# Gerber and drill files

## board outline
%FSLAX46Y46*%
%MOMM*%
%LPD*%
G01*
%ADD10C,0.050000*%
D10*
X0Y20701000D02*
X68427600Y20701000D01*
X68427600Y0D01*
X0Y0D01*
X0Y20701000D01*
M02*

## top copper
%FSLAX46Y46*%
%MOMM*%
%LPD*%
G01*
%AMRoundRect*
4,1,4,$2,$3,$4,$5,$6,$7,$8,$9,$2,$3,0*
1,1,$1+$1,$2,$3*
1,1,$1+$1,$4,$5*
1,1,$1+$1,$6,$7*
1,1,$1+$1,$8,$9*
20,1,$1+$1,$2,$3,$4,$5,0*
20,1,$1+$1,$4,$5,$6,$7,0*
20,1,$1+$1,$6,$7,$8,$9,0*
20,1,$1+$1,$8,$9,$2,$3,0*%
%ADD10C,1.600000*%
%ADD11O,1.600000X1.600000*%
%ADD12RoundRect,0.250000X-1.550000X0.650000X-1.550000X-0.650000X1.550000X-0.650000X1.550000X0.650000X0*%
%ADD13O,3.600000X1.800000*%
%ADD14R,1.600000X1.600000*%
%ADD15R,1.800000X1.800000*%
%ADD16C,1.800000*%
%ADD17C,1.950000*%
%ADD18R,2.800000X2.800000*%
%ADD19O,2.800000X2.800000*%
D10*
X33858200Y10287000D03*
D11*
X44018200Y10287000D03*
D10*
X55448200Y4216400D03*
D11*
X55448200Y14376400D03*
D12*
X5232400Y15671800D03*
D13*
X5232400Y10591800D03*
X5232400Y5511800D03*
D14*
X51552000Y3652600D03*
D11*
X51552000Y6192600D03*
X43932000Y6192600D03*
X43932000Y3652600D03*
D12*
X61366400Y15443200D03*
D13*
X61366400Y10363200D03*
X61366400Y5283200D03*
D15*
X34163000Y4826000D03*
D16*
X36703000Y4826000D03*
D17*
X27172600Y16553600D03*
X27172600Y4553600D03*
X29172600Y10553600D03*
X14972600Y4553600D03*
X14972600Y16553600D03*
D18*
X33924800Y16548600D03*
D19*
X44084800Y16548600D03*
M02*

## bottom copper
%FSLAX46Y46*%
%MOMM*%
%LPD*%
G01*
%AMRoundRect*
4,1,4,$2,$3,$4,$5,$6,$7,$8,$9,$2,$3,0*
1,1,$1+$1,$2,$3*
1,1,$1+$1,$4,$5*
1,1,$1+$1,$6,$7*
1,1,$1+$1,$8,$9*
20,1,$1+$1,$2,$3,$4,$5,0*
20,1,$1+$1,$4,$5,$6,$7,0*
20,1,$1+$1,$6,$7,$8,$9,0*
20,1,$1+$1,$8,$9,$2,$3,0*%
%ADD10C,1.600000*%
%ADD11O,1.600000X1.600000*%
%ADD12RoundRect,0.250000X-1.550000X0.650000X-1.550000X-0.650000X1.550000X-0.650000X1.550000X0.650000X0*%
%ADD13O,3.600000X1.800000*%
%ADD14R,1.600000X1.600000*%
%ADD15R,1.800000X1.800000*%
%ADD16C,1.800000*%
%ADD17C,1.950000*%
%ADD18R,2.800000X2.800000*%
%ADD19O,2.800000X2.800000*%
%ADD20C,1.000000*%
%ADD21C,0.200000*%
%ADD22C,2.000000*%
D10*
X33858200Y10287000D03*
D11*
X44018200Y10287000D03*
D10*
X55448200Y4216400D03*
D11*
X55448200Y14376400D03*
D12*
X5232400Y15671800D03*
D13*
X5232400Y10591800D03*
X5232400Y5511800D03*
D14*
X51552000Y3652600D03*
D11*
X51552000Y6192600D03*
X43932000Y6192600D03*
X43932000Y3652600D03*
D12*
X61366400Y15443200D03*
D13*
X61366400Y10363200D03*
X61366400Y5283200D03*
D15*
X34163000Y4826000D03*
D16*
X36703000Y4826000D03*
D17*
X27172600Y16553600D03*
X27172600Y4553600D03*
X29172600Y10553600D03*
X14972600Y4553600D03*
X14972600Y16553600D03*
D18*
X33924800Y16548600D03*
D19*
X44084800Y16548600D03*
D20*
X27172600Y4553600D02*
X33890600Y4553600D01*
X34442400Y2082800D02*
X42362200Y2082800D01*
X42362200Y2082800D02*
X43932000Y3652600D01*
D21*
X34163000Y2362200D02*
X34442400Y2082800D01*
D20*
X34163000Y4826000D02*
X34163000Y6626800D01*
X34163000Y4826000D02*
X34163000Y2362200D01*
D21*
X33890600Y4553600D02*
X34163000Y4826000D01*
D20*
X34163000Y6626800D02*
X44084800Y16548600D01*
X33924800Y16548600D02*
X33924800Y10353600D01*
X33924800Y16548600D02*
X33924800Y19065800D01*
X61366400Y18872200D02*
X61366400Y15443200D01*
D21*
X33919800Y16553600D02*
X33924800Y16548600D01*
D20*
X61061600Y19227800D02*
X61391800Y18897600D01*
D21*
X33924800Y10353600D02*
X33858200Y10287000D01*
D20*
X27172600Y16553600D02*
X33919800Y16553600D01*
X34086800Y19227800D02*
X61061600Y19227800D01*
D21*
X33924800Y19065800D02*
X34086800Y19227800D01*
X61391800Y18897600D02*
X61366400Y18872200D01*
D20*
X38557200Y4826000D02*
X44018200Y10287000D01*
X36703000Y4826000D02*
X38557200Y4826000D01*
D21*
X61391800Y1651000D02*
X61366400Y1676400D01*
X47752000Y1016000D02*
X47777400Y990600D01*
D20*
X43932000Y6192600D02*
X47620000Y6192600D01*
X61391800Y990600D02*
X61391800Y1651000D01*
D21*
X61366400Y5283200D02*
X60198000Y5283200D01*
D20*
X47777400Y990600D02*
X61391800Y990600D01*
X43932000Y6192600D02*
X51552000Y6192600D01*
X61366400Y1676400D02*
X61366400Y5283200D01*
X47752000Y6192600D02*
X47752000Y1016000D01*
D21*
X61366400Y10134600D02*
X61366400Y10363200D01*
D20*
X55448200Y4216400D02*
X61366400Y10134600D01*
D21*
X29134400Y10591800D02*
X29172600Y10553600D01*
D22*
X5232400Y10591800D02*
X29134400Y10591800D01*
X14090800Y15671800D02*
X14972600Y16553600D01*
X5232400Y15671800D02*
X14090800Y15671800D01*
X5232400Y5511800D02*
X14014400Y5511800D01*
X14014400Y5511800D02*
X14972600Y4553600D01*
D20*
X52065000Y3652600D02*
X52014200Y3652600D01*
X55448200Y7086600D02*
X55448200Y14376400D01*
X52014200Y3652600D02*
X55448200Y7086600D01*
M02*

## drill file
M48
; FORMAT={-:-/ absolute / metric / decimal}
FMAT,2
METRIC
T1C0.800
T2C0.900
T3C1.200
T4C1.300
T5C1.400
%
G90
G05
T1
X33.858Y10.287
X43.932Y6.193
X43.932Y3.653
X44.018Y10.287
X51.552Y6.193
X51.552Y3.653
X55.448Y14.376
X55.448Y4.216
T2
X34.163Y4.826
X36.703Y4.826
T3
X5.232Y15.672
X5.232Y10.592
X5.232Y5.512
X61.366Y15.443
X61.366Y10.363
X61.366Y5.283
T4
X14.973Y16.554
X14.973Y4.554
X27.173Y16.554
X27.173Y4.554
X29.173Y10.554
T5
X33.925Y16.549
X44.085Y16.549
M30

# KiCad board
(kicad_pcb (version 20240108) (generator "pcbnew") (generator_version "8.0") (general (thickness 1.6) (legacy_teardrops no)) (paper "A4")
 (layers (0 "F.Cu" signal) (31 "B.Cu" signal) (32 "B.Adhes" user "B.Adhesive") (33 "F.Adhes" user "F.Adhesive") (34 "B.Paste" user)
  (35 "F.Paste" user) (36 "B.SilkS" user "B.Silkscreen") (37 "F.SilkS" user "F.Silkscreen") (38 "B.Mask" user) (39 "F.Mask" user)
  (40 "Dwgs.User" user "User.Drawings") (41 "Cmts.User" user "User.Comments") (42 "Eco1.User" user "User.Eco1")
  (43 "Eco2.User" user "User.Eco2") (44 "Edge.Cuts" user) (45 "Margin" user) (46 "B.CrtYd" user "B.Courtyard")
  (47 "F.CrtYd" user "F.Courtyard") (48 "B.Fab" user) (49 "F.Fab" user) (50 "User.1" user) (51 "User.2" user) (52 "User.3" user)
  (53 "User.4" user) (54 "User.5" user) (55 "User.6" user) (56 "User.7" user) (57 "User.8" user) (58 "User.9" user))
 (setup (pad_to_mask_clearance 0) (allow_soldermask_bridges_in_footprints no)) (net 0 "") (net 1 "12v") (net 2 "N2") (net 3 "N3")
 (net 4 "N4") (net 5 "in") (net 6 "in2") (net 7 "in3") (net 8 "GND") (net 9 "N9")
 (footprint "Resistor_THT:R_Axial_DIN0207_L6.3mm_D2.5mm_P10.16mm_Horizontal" (layer "F.Cu") (at 33.8582 -10.287)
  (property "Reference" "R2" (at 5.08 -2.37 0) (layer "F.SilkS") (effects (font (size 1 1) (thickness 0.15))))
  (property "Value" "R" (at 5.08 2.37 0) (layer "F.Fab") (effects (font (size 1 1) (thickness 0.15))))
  (pad "1" thru_hole circle (at 0 0) (size 1.6 1.6) (drill 0.8) (layers "*.Cu" "*.Mask") (remove_unused_layers no) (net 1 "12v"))
  (pad "2" thru_hole oval (at 10.16 0) (size 1.6 1.6) (drill 0.8) (layers "*.Cu" "*.Mask") (remove_unused_layers no) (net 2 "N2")))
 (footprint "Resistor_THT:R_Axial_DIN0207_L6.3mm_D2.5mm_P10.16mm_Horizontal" (layer "F.Cu") (at 55.4482 -4.2164 90)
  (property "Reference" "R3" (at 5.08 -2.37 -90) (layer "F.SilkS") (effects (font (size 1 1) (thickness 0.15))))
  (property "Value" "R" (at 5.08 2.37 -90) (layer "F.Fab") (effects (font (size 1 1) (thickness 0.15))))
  (pad "1" thru_hole circle (at 0 0 90) (size 1.6 1.6) (drill 0.8) (layers "*.Cu" "*.Mask") (remove_unused_layers no) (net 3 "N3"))
  (pad "2" thru_hole oval (at 10.16 0 90) (size 1.6 1.6) (drill 0.8) (layers "*.Cu" "*.Mask") (remove_unused_layers no) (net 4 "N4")))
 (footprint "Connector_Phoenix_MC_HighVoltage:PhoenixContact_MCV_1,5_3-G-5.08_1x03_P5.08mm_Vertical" (layer "F.Cu") (at 5.2324 -15.6718 -90)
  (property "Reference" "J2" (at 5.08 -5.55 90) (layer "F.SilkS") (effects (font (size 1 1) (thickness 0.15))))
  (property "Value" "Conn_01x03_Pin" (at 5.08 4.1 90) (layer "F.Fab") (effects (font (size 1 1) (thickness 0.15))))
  (pad "1" thru_hole roundrect (at 0 0 270) (size 1.8 3.6) (drill 1.2) (layers "*.Cu" "*.Mask") (remove_unused_layers no)
   (roundrect_rratio 0.138889) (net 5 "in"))
  (pad "2" thru_hole oval (at 5.08 0 270) (size 1.8 3.6) (drill 1.2) (layers "*.Cu" "*.Mask") (remove_unused_layers no) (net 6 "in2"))
  (pad "3" thru_hole oval (at 10.16 0 270) (size 1.8 3.6) (drill 1.2) (layers "*.Cu" "*.Mask") (remove_unused_layers no) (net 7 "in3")))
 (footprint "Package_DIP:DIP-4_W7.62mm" (layer "F.Cu") (at 51.552 -3.6526 180)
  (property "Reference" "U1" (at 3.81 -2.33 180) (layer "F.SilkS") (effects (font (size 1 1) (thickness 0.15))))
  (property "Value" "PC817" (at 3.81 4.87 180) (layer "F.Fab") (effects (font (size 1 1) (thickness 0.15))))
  (pad "1" thru_hole rect (at 0 0 180) (size 1.6 1.6) (drill 0.8) (layers "*.Cu" "*.Mask") (remove_unused_layers no) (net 4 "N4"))
  (pad "2" thru_hole oval (at 0 2.54 180) (size 1.6 1.6) (drill 0.8) (layers "*.Cu" "*.Mask") (remove_unused_layers no) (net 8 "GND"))
  (pad "3" thru_hole oval (at 7.62 2.54 180) (size 1.6 1.6) (drill 0.8) (layers "*.Cu" "*.Mask") (remove_unused_layers no) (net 8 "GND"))
  (pad "4" thru_hole oval (at 7.62 0 180) (size 1.6 1.6) (drill 0.8) (layers "*.Cu" "*.Mask") (remove_unused_layers no) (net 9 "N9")))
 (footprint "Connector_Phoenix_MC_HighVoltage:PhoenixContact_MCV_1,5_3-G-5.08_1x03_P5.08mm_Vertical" (layer "F.Cu")
  (at 61.3664 -15.4432 -90)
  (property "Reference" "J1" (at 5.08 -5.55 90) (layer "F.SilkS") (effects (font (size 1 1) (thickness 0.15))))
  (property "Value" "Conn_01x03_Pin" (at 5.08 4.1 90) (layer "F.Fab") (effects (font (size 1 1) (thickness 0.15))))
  (pad "1" thru_hole roundrect (at 0 0 270) (size 1.8 3.6) (drill 1.2) (layers "*.Cu" "*.Mask") (remove_unused_layers no)
   (roundrect_rratio 0.138889) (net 1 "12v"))
  (pad "2" thru_hole oval (at 5.08 0 270) (size 1.8 3.6) (drill 1.2) (layers "*.Cu" "*.Mask") (remove_unused_layers no) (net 3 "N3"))
  (pad "3" thru_hole oval (at 10.16 0 270) (size 1.8 3.6) (drill 1.2) (layers "*.Cu" "*.Mask") (remove_unused_layers no) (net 8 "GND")))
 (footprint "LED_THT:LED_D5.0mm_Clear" (layer "F.Cu") (at 34.163 -4.826)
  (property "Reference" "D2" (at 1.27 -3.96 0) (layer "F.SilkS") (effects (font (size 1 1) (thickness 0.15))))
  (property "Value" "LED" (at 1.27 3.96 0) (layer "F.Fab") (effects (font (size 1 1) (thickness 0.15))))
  (pad "1" thru_hole rect (at 0 0) (size 1.8 1.8) (drill 0.9) (layers "*.Cu" "*.Mask") (remove_unused_layers no) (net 9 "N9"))
  (pad "2" thru_hole circle (at 2.54 0) (size 1.8 1.8) (drill 0.9) (layers "*.Cu" "*.Mask") (remove_unused_layers no) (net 2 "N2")))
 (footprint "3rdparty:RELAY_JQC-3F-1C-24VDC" (layer "F.Cu") (at 21.0726 -10.5536)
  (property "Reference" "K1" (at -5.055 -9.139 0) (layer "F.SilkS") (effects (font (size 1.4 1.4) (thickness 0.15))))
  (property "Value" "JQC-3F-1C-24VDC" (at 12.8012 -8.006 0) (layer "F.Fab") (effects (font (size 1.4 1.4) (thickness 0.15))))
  (pad "COIL1" thru_hole circle (at 6.1 -6) (size 1.95 1.95) (drill 1.3) (layers "*.Cu" "*.Mask") (remove_unused_layers no) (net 1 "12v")
   (solder_mask_margin 0.102))
  (pad "COIL2" thru_hole circle (at 6.1 6) (size 1.95 1.95) (drill 1.3) (layers "*.Cu" "*.Mask") (remove_unused_layers no) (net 9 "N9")
   (solder_mask_margin 0.102))
  (pad "COM" thru_hole circle (at 8.1 0) (size 1.95 1.95) (drill 1.3) (layers "*.Cu" "*.Mask") (remove_unused_layers no) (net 6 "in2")
   (solder_mask_margin 0.102))
  (pad "NC" thru_hole circle (at -6.1 6) (size 1.95 1.95) (drill 1.3) (layers "*.Cu" "*.Mask") (remove_unused_layers no) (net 7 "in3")
   (solder_mask_margin 0.102))
  (pad "NO" thru_hole circle (at -6.1 -6) (size 1.95 1.95) (drill 1.3) (layers "*.Cu" "*.Mask") (remove_unused_layers no) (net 5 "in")
   (solder_mask_margin 0.102)))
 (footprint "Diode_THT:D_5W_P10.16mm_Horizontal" (layer "F.Cu") (at 33.9248 -16.5486)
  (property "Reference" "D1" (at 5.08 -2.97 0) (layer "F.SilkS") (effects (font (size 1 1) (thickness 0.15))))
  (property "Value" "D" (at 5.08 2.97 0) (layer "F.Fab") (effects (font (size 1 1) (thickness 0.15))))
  (pad "1" thru_hole rect (at 0 0) (size 2.8 2.8) (drill 1.4) (layers "*.Cu" "*.Mask") (remove_unused_layers no) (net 1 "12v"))
  (pad "2" thru_hole oval (at 10.16 0) (size 2.8 2.8) (drill 1.4) (layers "*.Cu" "*.Mask") (remove_unused_layers no) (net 9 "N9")))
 (gr_rect (start 0 -20.701) (end 68.4276 0) (stroke (width 0.05) (type default)) (fill none) (layer "Edge.Cuts"))
 (segment (start 27.1726 -4.5536) (end 33.8906 -4.5536) (width 1) (layer "B.Cu") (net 9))
 (segment (start 34.4424 -2.0828) (end 42.3622 -2.0828) (width 1) (layer "B.Cu") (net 9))
 (segment (start 42.3622 -2.0828) (end 43.932 -3.6526) (width 1) (layer "B.Cu") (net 9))
 (segment (start 34.163 -2.3622) (end 34.4424 -2.0828) (width 0.2) (layer "B.Cu") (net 9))
 (segment (start 34.163 -4.826) (end 34.163 -6.6268) (width 1) (layer "B.Cu") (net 9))
 (segment (start 34.163 -4.826) (end 34.163 -2.3622) (width 1) (layer "B.Cu") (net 9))
 (segment (start 33.8906 -4.5536) (end 34.163 -4.826) (width 0.2) (layer "B.Cu") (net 9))
 (segment (start 34.163 -6.6268) (end 44.0848 -16.5486) (width 1) (layer "B.Cu") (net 9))
 (segment (start 33.9248 -16.5486) (end 33.9248 -10.3536) (width 1) (layer "B.Cu") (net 1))
 (segment (start 33.9248 -16.5486) (end 33.9248 -19.0658) (width 1) (layer "B.Cu") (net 1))
 (segment (start 61.3664 -18.8722) (end 61.3664 -15.4432) (width 1) (layer "B.Cu") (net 1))
 (segment (start 33.9198 -16.5536) (end 33.9248 -16.5486) (width 0.2) (layer "B.Cu") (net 1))
 (segment (start 61.0616 -19.2278) (end 61.3918 -18.8976) (width 1) (layer "B.Cu") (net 1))
 (segment (start 33.9248 -10.3536) (end 33.8582 -10.287) (width 0.2) (layer "B.Cu") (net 1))
 (segment (start 27.1726 -16.5536) (end 33.9198 -16.5536) (width 1) (layer "B.Cu") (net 1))
 (segment (start 34.0868 -19.2278) (end 61.0616 -19.2278) (width 1) (layer "B.Cu") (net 1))
 (segment (start 33.9248 -19.0658) (end 34.0868 -19.2278) (width 0.2) (layer "B.Cu") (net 1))
 (segment (start 61.3918 -18.8976) (end 61.3664 -18.8722) (width 0.2) (layer "B.Cu") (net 1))
 (segment (start 38.5572 -4.826) (end 44.0182 -10.287) (width 1) (layer "B.Cu") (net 2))
 (segment (start 36.703 -4.826) (end 38.5572 -4.826) (width 1) (layer "B.Cu") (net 2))
 (segment (start 61.3918 -1.651) (end 61.3664 -1.6764) (width 0.2) (layer "B.Cu") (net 8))
 (segment (start 47.752 -1.016) (end 47.7774 -0.9906) (width 0.2) (layer "B.Cu") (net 8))
 (segment (start 43.932 -6.1926) (end 47.62 -6.1926) (width 1) (layer "B.Cu") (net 8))
 (segment (start 61.3918 -0.9906) (end 61.3918 -1.651) (width 1) (layer "B.Cu") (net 8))
 (segment (start 61.3664 -5.2832) (end 60.198 -5.2832) (width 0.2) (layer "B.Cu") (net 8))
 (segment (start 47.7774 -0.9906) (end 61.3918 -0.9906) (width 1) (layer "B.Cu") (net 8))
 (segment (start 43.932 -6.1926) (end 51.552 -6.1926) (width 1) (layer "B.Cu") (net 8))
 (segment (start 61.3664 -1.6764) (end 61.3664 -5.2832) (width 1) (layer "B.Cu") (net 8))
 (segment (start 47.752 -6.1926) (end 47.752 -1.016) (width 1) (layer "B.Cu") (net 8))
 (segment (start 61.3664 -10.1346) (end 61.3664 -10.3632) (width 0.2) (layer "B.Cu") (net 3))
 (segment (start 55.4482 -4.2164) (end 61.3664 -10.1346) (width 1) (layer "B.Cu") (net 3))
 (segment (start 29.1344 -10.5918) (end 29.1726 -10.5536) (width 0.2) (layer "B.Cu") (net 6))
 (segment (start 5.2324 -10.5918) (end 29.1344 -10.5918) (width 2) (layer "B.Cu") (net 6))
 (segment (start 14.0908 -15.6718) (end 14.9726 -16.5536) (width 2) (layer "B.Cu") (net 5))
 (segment (start 5.2324 -15.6718) (end 14.0908 -15.6718) (width 2) (layer "B.Cu") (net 5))
 (segment (start 5.2324 -5.5118) (end 14.0144 -5.5118) (width 2) (layer "B.Cu") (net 7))
 (segment (start 14.0144 -5.5118) (end 14.9726 -4.5536) (width 2) (layer "B.Cu") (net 7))
 (segment (start 52.065 -3.6526) (end 52.0142 -3.6526) (width 1) (layer "B.Cu") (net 4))
 (segment (start 55.4482 -7.0866) (end 55.4482 -14.3764) (width 1) (layer "B.Cu") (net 4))
 (segment (start 52.0142 -3.6526) (end 55.4482 -7.0866) (width 1) (layer "B.Cu") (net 4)))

